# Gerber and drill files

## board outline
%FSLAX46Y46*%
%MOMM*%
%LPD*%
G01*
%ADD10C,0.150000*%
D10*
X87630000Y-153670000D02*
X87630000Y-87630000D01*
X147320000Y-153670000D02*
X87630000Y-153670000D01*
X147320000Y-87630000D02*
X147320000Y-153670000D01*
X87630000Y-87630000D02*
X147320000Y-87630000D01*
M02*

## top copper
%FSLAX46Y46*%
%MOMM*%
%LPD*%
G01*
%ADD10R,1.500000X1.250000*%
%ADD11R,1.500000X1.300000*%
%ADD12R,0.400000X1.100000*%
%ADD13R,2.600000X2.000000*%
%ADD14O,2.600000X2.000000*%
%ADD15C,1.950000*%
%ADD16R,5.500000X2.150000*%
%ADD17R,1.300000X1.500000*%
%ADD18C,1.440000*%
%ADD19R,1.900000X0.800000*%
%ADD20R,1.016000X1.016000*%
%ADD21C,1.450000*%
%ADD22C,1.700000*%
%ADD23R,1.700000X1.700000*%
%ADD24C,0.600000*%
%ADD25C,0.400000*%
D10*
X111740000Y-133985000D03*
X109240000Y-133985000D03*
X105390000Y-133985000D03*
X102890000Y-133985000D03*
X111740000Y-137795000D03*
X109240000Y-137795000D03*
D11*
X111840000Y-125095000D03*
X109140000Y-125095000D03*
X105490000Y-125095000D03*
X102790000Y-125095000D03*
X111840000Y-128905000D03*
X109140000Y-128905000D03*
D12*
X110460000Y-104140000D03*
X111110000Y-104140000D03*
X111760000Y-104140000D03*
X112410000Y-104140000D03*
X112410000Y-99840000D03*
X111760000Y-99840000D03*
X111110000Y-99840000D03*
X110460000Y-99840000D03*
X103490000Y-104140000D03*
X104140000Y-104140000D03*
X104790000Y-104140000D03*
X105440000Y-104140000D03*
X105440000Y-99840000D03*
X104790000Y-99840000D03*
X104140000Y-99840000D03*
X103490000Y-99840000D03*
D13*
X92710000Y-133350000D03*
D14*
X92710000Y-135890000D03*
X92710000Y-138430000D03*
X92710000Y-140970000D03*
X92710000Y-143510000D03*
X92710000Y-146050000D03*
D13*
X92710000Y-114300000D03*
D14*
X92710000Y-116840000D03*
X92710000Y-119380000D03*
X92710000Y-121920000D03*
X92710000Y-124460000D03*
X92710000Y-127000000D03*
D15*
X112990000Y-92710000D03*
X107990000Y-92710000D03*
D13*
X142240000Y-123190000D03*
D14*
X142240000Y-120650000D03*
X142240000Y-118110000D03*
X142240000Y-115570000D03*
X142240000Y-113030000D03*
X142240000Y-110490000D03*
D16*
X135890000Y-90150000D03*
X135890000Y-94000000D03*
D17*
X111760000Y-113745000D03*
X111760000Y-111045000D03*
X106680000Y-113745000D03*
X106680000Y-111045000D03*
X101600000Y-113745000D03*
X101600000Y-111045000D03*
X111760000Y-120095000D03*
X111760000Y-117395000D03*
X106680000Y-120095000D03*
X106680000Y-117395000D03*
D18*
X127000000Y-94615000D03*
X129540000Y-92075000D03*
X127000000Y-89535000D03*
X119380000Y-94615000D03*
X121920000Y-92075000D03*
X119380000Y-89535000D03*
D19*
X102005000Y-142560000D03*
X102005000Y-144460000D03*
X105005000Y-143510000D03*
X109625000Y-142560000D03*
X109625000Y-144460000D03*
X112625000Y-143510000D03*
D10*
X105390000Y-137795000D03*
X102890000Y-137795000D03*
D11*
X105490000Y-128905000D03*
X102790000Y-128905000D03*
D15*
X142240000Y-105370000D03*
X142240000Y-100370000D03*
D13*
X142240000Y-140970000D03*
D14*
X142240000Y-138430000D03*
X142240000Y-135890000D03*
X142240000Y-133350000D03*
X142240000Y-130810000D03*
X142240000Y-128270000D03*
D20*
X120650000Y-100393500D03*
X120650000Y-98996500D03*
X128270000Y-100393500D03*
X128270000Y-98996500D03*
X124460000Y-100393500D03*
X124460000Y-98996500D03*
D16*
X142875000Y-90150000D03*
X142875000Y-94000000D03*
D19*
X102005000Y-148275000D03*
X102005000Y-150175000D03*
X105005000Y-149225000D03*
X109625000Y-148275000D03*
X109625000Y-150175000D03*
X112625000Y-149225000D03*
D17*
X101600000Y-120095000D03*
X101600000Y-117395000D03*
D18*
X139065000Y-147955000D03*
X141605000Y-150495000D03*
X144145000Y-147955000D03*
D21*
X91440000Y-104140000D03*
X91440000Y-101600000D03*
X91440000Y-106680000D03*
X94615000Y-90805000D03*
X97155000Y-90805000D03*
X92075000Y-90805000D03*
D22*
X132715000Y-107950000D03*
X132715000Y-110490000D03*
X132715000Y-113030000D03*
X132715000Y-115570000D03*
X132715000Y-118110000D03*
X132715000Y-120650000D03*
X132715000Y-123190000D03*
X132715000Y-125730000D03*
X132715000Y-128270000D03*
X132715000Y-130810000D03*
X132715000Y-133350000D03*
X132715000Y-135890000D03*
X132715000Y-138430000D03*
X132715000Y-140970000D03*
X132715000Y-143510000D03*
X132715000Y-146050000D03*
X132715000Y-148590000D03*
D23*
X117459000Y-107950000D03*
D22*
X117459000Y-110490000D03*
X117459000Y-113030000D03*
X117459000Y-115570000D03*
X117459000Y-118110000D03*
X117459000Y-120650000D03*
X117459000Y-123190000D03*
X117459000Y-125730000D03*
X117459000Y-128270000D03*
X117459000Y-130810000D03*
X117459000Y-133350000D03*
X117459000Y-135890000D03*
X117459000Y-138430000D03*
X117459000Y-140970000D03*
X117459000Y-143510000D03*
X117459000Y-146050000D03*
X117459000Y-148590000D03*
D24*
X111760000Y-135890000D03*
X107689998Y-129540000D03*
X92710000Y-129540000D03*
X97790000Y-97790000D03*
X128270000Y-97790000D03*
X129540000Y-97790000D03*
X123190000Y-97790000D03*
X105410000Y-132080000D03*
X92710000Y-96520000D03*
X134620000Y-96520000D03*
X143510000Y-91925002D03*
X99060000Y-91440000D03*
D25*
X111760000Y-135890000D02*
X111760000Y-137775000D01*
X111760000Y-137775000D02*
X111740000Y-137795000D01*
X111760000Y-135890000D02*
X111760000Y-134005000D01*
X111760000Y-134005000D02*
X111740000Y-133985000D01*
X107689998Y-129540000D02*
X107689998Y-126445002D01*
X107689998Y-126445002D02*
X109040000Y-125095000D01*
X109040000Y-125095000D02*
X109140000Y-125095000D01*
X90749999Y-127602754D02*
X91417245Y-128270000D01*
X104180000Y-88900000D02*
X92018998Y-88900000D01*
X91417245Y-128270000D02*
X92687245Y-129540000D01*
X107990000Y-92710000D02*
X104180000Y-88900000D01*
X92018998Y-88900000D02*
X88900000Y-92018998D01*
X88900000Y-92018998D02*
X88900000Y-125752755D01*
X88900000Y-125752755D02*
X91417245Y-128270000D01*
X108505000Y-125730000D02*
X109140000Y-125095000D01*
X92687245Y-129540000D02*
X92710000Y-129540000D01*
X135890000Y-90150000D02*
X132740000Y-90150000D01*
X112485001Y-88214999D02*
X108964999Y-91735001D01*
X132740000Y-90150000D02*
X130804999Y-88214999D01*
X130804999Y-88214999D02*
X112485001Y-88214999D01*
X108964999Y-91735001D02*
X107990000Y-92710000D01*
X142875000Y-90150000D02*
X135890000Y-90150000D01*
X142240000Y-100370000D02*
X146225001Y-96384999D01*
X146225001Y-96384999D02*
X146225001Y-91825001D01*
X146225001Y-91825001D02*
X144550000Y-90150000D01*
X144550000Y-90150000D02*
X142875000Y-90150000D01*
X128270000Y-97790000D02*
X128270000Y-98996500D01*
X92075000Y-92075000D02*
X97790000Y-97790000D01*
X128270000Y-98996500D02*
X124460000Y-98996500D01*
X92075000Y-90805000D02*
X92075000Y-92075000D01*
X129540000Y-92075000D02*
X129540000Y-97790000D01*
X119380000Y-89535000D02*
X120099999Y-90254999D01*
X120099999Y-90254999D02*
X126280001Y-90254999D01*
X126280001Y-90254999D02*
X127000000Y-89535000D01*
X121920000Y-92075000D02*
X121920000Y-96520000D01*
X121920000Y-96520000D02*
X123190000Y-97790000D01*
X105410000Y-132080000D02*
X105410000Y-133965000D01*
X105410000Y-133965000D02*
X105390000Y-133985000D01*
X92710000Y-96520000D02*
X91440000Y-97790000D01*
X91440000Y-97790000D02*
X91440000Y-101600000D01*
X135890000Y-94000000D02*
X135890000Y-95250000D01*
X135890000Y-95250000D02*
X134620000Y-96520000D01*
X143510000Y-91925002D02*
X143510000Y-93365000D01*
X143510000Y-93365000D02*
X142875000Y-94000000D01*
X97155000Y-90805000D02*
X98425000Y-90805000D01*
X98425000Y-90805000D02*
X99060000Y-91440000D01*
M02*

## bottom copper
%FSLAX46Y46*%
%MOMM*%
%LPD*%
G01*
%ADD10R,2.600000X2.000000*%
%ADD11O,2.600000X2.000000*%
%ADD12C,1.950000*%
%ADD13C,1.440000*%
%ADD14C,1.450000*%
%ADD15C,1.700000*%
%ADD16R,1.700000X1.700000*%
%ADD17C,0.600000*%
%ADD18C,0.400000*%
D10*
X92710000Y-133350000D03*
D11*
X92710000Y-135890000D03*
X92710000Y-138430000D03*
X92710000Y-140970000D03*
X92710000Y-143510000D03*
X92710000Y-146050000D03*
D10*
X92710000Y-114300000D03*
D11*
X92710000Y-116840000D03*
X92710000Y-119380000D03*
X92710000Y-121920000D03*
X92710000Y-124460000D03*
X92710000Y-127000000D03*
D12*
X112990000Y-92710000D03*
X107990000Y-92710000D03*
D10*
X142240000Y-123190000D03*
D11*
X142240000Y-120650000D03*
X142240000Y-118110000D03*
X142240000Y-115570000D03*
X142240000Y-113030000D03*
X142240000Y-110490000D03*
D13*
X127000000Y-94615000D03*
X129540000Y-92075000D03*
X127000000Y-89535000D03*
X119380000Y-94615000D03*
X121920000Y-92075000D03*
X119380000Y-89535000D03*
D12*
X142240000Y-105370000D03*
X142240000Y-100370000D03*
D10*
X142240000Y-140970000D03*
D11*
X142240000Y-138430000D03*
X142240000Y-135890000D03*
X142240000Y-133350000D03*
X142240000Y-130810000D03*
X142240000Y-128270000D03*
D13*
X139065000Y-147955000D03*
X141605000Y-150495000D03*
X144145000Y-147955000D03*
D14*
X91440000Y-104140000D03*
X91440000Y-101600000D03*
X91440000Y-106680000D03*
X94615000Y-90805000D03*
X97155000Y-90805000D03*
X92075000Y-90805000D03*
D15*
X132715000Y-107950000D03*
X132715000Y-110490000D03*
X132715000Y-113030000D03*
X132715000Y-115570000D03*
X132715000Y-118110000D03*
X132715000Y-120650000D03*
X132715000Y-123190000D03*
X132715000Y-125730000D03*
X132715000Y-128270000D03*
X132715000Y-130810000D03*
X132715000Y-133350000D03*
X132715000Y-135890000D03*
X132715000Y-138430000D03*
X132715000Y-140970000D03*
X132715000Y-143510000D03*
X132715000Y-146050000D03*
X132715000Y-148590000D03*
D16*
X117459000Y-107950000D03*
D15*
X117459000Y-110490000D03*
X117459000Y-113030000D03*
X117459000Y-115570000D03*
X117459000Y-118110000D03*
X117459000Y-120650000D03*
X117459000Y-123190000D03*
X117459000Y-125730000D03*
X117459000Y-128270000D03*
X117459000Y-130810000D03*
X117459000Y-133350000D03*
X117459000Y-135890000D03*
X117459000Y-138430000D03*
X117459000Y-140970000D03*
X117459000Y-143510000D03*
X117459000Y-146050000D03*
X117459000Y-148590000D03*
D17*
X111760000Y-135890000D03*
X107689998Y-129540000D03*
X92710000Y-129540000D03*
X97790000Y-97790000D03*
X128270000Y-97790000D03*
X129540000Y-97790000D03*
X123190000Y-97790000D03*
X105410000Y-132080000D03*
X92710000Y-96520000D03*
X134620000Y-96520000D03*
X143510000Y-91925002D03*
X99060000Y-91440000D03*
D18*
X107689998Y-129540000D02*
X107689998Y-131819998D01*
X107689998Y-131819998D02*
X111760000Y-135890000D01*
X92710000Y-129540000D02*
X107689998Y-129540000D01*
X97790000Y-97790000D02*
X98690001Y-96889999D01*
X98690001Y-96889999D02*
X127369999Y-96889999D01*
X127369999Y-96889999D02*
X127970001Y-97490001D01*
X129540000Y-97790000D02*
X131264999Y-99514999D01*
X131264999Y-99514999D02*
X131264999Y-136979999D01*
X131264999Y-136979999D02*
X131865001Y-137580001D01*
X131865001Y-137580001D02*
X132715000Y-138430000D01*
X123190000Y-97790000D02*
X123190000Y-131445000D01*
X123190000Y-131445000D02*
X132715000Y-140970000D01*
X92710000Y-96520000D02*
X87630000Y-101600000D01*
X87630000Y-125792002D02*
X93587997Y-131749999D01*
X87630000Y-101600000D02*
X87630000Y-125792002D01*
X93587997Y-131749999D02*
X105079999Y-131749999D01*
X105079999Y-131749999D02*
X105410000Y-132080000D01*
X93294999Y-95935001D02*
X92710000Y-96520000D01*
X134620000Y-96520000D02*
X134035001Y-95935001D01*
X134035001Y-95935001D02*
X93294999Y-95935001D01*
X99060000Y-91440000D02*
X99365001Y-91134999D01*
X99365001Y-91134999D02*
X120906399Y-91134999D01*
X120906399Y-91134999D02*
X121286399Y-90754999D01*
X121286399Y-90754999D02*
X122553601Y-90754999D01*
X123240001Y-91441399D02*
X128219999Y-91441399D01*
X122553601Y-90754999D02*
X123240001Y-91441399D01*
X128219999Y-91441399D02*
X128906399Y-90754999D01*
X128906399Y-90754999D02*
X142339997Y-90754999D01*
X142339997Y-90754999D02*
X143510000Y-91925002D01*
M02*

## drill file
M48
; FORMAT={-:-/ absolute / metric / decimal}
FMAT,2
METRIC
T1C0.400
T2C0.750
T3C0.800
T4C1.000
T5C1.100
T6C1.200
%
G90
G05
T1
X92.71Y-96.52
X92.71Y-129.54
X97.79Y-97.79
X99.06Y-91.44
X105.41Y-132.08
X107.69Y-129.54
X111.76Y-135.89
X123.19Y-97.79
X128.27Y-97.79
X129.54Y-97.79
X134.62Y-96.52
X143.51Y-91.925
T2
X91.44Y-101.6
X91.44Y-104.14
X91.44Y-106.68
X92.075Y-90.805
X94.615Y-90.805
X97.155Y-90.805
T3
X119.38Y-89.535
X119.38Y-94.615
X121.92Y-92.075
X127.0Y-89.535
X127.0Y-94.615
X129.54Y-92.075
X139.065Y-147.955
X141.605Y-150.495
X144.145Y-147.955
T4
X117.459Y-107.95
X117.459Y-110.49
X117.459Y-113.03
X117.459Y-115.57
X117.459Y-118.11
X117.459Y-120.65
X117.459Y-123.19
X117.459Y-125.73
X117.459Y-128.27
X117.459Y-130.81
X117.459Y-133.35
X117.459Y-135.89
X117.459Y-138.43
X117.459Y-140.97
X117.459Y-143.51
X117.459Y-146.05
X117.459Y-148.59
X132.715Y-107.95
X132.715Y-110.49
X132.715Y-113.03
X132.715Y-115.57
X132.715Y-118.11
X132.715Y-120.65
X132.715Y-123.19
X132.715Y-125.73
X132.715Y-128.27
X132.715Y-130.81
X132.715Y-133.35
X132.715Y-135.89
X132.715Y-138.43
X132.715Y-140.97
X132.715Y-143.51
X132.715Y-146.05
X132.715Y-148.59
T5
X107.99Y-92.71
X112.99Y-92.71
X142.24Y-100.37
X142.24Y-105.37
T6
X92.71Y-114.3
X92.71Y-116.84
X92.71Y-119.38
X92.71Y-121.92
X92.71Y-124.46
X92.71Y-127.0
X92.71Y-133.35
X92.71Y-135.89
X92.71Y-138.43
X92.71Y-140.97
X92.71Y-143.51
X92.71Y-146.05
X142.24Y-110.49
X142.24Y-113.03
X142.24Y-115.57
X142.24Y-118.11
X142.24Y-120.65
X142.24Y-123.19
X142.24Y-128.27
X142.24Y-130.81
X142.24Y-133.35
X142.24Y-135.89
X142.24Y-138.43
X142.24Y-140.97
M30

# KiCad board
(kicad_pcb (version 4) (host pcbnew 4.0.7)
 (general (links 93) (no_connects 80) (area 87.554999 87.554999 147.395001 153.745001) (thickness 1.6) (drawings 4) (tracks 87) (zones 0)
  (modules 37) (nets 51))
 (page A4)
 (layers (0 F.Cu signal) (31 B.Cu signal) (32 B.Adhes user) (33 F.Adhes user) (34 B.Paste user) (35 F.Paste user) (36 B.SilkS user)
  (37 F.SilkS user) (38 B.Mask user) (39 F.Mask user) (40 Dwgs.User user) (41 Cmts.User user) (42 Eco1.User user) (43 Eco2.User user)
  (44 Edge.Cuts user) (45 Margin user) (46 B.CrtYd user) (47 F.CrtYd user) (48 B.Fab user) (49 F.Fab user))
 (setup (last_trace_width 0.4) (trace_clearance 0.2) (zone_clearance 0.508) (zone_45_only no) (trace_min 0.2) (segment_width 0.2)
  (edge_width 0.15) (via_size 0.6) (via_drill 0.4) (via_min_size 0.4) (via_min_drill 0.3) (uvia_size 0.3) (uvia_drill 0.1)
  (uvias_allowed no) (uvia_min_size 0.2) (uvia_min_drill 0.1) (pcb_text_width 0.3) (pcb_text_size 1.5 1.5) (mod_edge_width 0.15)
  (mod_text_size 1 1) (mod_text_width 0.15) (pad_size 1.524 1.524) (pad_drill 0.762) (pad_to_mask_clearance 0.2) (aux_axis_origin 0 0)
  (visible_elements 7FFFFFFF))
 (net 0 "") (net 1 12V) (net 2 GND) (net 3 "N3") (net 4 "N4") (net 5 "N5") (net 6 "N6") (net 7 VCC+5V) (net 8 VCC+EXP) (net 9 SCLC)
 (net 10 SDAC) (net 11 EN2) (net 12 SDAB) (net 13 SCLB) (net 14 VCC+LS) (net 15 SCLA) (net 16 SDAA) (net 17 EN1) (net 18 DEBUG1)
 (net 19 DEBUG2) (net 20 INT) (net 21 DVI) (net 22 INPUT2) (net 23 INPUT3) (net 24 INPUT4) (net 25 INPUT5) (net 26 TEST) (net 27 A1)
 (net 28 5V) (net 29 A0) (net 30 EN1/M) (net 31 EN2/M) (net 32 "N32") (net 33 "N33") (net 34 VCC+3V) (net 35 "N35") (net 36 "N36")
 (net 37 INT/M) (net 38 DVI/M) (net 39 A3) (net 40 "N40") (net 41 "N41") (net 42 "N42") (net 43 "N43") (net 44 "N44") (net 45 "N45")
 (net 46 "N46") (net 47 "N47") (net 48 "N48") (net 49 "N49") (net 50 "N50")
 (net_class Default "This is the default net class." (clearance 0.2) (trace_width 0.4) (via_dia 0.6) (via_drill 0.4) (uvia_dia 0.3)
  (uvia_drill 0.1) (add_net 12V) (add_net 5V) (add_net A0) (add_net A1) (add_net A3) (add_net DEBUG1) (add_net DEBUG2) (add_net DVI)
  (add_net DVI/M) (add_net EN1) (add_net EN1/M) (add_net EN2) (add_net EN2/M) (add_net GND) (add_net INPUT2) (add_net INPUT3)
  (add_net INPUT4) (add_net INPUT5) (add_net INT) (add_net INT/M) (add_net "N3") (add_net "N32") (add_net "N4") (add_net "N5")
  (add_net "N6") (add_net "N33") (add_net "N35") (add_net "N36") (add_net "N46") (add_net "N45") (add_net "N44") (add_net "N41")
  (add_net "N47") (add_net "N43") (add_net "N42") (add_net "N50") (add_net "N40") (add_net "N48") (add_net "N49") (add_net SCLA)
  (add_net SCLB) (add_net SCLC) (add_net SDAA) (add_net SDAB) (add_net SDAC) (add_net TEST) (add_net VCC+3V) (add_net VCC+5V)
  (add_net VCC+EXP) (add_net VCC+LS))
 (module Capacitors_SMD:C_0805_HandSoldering (layer F.Cu) (at 110.49 133.985 180)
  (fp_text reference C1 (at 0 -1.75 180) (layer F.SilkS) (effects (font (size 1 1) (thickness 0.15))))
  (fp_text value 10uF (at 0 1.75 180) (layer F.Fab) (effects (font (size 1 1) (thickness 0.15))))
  (pad 1 smd rect (at -1.25 0 180) (size 1.5 1.25) (layers F.Cu F.Paste F.Mask) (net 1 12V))
  (pad 2 smd rect (at 1.25 0 180) (size 1.5 1.25) (layers F.Cu F.Paste F.Mask) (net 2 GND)))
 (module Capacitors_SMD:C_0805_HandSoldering (layer F.Cu) (at 104.14 133.985 180)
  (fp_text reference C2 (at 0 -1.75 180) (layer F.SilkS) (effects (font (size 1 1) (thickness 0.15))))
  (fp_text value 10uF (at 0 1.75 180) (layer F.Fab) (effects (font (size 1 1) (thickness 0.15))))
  (pad 1 smd rect (at -1.25 0 180) (size 1.5 1.25) (layers F.Cu F.Paste F.Mask) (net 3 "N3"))
  (pad 2 smd rect (at 1.25 0 180) (size 1.5 1.25) (layers F.Cu F.Paste F.Mask) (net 2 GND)))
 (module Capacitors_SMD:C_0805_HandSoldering (layer F.Cu) (at 110.49 137.795 180)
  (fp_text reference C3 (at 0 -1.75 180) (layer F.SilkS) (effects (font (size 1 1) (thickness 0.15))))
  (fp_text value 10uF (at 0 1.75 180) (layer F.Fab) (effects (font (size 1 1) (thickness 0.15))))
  (pad 1 smd rect (at -1.25 0 180) (size 1.5 1.25) (layers F.Cu F.Paste F.Mask) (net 1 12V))
  (pad 2 smd rect (at 1.25 0 180) (size 1.5 1.25) (layers F.Cu F.Paste F.Mask) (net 2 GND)))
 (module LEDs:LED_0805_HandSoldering (layer F.Cu) (at 110.49 125.095 180)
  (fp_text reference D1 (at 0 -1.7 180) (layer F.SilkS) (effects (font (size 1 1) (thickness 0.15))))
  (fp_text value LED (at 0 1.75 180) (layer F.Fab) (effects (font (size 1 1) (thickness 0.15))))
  (pad 1 smd rect (at -1.35 0 180) (size 1.5 1.3) (layers F.Cu F.Paste F.Mask) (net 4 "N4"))
  (pad 2 smd rect (at 1.35 0 180) (size 1.5 1.3) (layers F.Cu F.Paste F.Mask) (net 1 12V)))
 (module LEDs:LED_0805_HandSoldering (layer F.Cu) (at 104.14 125.095 180)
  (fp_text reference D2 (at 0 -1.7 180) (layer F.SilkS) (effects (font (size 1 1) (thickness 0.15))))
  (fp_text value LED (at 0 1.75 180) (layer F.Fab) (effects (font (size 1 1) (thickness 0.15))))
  (pad 1 smd rect (at -1.35 0 180) (size 1.5 1.3) (layers F.Cu F.Paste F.Mask) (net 2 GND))
  (pad 2 smd rect (at 1.35 0 180) (size 1.5 1.3) (layers F.Cu F.Paste F.Mask) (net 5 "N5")))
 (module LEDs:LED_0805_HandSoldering (layer F.Cu) (at 110.49 128.905 180)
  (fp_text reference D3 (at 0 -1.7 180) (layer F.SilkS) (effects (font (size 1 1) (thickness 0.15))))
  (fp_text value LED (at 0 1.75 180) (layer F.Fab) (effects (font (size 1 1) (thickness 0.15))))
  (pad 1 smd rect (at -1.35 0 180) (size 1.5 1.3) (layers F.Cu F.Paste F.Mask) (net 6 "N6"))
  (pad 2 smd rect (at 1.35 0 180) (size 1.5 1.3) (layers F.Cu F.Paste F.Mask) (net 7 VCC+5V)))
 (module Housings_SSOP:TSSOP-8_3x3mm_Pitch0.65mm (layer F.Cu) (at 111.435 101.99 90)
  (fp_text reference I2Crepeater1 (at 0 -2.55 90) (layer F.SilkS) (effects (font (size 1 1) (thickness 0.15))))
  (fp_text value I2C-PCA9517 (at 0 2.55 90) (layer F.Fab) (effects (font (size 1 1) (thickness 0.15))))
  (pad 1 smd rect (at -2.15 -0.975 90) (size 1.1 0.4) (layers F.Cu F.Paste F.Mask) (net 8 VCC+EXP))
  (pad 2 smd rect (at -2.15 -0.325 90) (size 1.1 0.4) (layers F.Cu F.Paste F.Mask) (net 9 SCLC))
  (pad 3 smd rect (at -2.15 0.325 90) (size 1.1 0.4) (layers F.Cu F.Paste F.Mask) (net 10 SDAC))
  (pad 4 smd rect (at -2.15 0.975 90) (size 1.1 0.4) (layers F.Cu F.Paste F.Mask) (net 2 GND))
  (pad 5 smd rect (at 2.15 0.975 90) (size 1.1 0.4) (layers F.Cu F.Paste F.Mask) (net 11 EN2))
  (pad 6 smd rect (at 2.15 0.325 90) (size 1.1 0.4) (layers F.Cu F.Paste F.Mask) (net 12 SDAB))
  (pad 7 smd rect (at 2.15 -0.325 90) (size 1.1 0.4) (layers F.Cu F.Paste F.Mask) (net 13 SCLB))
  (pad 8 smd rect (at 2.15 -0.975 90) (size 1.1 0.4) (layers F.Cu F.Paste F.Mask) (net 7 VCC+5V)))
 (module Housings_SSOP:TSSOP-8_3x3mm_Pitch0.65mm (layer F.Cu) (at 104.465 101.99 90)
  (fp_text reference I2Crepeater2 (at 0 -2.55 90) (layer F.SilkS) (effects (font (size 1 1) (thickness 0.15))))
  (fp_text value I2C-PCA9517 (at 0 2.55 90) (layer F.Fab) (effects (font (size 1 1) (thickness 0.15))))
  (pad 1 smd rect (at -2.15 -0.975 90) (size 1.1 0.4) (layers F.Cu F.Paste F.Mask) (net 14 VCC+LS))
  (pad 2 smd rect (at -2.15 -0.325 90) (size 1.1 0.4) (layers F.Cu F.Paste F.Mask) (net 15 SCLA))
  (pad 3 smd rect (at -2.15 0.325 90) (size 1.1 0.4) (layers F.Cu F.Paste F.Mask) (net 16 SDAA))
  (pad 4 smd rect (at -2.15 0.975 90) (size 1.1 0.4) (layers F.Cu F.Paste F.Mask) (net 2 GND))
  (pad 5 smd rect (at 2.15 0.975 90) (size 1.1 0.4) (layers F.Cu F.Paste F.Mask) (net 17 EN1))
  (pad 6 smd rect (at 2.15 0.325 90) (size 1.1 0.4) (layers F.Cu F.Paste F.Mask) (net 12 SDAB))
  (pad 7 smd rect (at 2.15 -0.325 90) (size 1.1 0.4) (layers F.Cu F.Paste F.Mask) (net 13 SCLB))
  (pad 8 smd rect (at 2.15 -0.975 90) (size 1.1 0.4) (layers F.Cu F.Paste F.Mask) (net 7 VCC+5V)))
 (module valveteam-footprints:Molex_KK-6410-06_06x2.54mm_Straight (layer F.Cu) (at 92.71 133.35 270)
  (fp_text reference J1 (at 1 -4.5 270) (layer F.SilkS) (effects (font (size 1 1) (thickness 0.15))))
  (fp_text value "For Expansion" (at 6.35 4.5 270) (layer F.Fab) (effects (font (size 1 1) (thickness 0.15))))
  (pad 1 thru_hole rect (at 0 0 270) (size 2 2.6) (drill 1.2) (layers *.Cu *.Mask) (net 8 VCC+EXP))
  (pad 2 thru_hole oval (at 2.54 0 270) (size 2 2.6) (drill 1.2) (layers *.Cu *.Mask) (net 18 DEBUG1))
  (pad 3 thru_hole oval (at 5.08 0 270) (size 2 2.6) (drill 1.2) (layers *.Cu *.Mask) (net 10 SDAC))
  (pad 4 thru_hole oval (at 7.62 0 270) (size 2 2.6) (drill 1.2) (layers *.Cu *.Mask) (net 9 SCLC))
  (pad 5 thru_hole oval (at 10.16 0 270) (size 2 2.6) (drill 1.2) (layers *.Cu *.Mask) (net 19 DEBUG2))
  (pad 6 thru_hole oval (at 12.7 0 270) (size 2 2.6) (drill 1.2) (layers *.Cu *.Mask) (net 2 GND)))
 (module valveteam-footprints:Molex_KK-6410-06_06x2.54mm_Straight (layer F.Cu) (at 92.71 114.3 270)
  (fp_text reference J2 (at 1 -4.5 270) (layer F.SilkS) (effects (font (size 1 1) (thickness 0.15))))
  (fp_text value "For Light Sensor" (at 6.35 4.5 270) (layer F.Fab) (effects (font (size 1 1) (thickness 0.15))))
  (pad 1 thru_hole rect (at 0 0 270) (size 2 2.6) (drill 1.2) (layers *.Cu *.Mask) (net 14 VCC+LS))
  (pad 2 thru_hole oval (at 2.54 0 270) (size 2 2.6) (drill 1.2) (layers *.Cu *.Mask) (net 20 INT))
  (pad 3 thru_hole oval (at 5.08 0 270) (size 2 2.6) (drill 1.2) (layers *.Cu *.Mask) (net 16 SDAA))
  (pad 4 thru_hole oval (at 7.62 0 270) (size 2 2.6) (drill 1.2) (layers *.Cu *.Mask) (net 15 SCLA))
  (pad 5 thru_hole oval (at 10.16 0 270) (size 2 2.6) (drill 1.2) (layers *.Cu *.Mask) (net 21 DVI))
  (pad 6 thru_hole oval (at 12.7 0 270) (size 2 2.6) (drill 1.2) (layers *.Cu *.Mask) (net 2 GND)))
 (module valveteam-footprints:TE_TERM (layer F.Cu) (at 110.49 92.71)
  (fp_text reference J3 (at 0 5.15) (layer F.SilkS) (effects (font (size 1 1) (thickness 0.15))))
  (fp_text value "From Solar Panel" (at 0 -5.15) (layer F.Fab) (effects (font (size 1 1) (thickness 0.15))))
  (pad 2 thru_hole circle (at 2.5 0) (size 1.95 1.95) (drill 1.1) (layers *.Cu *.Mask F.SilkS) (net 2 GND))
  (pad 1 thru_hole circle (at -2.5 0) (size 1.95 1.95) (drill 1.1) (layers *.Cu *.Mask F.SilkS) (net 1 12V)))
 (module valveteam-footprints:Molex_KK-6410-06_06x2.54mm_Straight (layer F.Cu) (at 142.24 123.19 90)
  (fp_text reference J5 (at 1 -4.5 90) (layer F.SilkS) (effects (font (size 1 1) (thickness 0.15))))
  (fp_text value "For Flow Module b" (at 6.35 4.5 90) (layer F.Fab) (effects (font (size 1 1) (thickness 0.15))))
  (pad 1 thru_hole rect (at 0 0 90) (size 2 2.6) (drill 1.2) (layers *.Cu *.Mask) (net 7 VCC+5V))
  (pad 2 thru_hole oval (at 2.54 0 90) (size 2 2.6) (drill 1.2) (layers *.Cu *.Mask) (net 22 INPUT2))
  (pad 3 thru_hole oval (at 5.08 0 90) (size 2 2.6) (drill 1.2) (layers *.Cu *.Mask) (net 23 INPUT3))
  (pad 4 thru_hole oval (at 7.62 0 90) (size 2 2.6) (drill 1.2) (layers *.Cu *.Mask) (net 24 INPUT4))
  (pad 5 thru_hole oval (at 10.16 0 90) (size 2 2.6) (drill 1.2) (layers *.Cu *.Mask) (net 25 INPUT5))
  (pad 6 thru_hole oval (at 12.7 0 90) (size 2 2.6) (drill 1.2) (layers *.Cu *.Mask) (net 2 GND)))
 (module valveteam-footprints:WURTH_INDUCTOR (layer F.Cu) (at 135.89 92.075)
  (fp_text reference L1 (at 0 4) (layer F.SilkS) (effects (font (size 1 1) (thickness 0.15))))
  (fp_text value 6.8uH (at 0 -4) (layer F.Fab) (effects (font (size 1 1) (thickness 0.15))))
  (pad 1 smd rect (at 0 -1.925) (size 5.5 2.15) (layers F.Cu F.Paste F.Mask) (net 1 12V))
  (pad 2 smd rect (at 0 1.925) (size 5.5 2.15) (layers F.Cu F.Paste F.Mask) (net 3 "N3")))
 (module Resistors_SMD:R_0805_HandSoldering (layer F.Cu) (at 111.76 112.395 90)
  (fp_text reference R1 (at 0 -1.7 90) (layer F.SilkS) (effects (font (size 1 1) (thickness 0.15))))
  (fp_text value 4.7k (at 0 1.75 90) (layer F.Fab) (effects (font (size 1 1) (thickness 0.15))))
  (pad 1 smd rect (at -1.35 0 90) (size 1.5 1.3) (layers F.Cu F.Paste F.Mask) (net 7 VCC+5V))
  (pad 2 smd rect (at 1.35 0 90) (size 1.5 1.3) (layers F.Cu F.Paste F.Mask) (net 13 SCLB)))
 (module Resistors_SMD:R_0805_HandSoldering (layer F.Cu) (at 106.68 112.395 90)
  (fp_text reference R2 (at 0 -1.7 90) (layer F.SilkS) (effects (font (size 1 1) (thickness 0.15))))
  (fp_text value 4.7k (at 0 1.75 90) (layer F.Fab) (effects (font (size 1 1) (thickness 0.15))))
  (pad 1 smd rect (at -1.35 0 90) (size 1.5 1.3) (layers F.Cu F.Paste F.Mask) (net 7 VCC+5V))
  (pad 2 smd rect (at 1.35 0 90) (size 1.5 1.3) (layers F.Cu F.Paste F.Mask) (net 12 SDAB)))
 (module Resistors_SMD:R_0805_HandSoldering (layer F.Cu) (at 101.6 112.395 90)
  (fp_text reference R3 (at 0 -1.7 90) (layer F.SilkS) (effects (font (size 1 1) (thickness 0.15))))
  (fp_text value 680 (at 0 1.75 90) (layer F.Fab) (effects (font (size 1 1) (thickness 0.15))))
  (pad 1 smd rect (at -1.35 0 90) (size 1.5 1.3) (layers F.Cu F.Paste F.Mask) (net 4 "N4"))
  (pad 2 smd rect (at 1.35 0 90) (size 1.5 1.3) (layers F.Cu F.Paste F.Mask) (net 2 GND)))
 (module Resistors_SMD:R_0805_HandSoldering (layer F.Cu) (at 111.76 118.745 90)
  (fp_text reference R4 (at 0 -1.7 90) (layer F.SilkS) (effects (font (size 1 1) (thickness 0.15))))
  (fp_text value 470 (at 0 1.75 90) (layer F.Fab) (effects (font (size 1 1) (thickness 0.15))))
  (pad 1 smd rect (at -1.35 0 90) (size 1.5 1.3) (layers F.Cu F.Paste F.Mask) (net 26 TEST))
  (pad 2 smd rect (at 1.35 0 90) (size 1.5 1.3) (layers F.Cu F.Paste F.Mask) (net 5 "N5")))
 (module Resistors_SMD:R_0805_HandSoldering (layer F.Cu) (at 106.68 118.745 90)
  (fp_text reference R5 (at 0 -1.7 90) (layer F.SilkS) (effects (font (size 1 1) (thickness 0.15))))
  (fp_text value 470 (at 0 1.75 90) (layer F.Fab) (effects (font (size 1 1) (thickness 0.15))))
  (pad 1 smd rect (at -1.35 0 90) (size 1.5 1.3) (layers F.Cu F.Paste F.Mask) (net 6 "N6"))
  (pad 2 smd rect (at 1.35 0 90) (size 1.5 1.3) (layers F.Cu F.Paste F.Mask) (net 2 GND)))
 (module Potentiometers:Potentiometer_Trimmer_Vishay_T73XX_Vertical (layer F.Cu) (at 127 89.535)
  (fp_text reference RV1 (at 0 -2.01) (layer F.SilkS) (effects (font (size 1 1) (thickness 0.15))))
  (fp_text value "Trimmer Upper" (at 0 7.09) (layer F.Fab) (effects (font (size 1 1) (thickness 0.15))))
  (pad 3 thru_hole circle (at 0 5.08) (size 1.44 1.44) (drill 0.8) (layers *.Cu *.Mask) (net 2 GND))
  (pad 2 thru_hole circle (at 2.54 2.54) (size 1.44 1.44) (drill 0.8) (layers *.Cu *.Mask) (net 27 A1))
  (pad 1 thru_hole circle (at 0 0) (size 1.44 1.44) (drill 0.8) (layers *.Cu *.Mask) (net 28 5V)))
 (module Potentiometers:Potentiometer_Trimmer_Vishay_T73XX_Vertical (layer F.Cu) (at 119.38 89.535)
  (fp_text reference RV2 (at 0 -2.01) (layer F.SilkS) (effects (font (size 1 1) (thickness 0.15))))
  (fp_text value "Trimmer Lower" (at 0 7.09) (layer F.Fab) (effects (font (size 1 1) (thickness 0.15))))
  (pad 3 thru_hole circle (at 0 5.08) (size 1.44 1.44) (drill 0.8) (layers *.Cu *.Mask) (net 2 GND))
  (pad 2 thru_hole circle (at 2.54 2.54) (size 1.44 1.44) (drill 0.8) (layers *.Cu *.Mask) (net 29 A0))
  (pad 1 thru_hole circle (at 0 0) (size 1.44 1.44) (drill 0.8) (layers *.Cu *.Mask) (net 28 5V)))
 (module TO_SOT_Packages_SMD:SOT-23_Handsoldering (layer F.Cu) (at 103.505 143.51)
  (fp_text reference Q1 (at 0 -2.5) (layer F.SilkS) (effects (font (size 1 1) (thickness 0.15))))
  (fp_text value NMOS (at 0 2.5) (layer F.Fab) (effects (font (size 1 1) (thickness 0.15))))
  (pad 1 smd rect (at -1.5 -0.95) (size 1.9 0.8) (layers F.Cu F.Paste F.Mask) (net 17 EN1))
  (pad 2 smd rect (at -1.5 0.95) (size 1.9 0.8) (layers F.Cu F.Paste F.Mask) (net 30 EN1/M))
  (pad 3 smd rect (at 1.5 0) (size 1.9 0.8) (layers F.Cu F.Paste F.Mask) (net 2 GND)))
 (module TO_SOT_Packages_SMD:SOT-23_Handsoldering (layer F.Cu) (at 111.125 143.51)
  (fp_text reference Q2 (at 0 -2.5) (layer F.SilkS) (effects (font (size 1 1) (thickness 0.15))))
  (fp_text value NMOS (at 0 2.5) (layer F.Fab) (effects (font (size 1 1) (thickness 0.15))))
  (pad 1 smd rect (at -1.5 -0.95) (size 1.9 0.8) (layers F.Cu F.Paste F.Mask) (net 11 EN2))
  (pad 2 smd rect (at -1.5 0.95) (size 1.9 0.8) (layers F.Cu F.Paste F.Mask) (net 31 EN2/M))
  (pad 3 smd rect (at 1.5 0) (size 1.9 0.8) (layers F.Cu F.Paste F.Mask) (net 2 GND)))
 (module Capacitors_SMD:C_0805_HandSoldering (layer F.Cu) (at 104.14 137.795 180)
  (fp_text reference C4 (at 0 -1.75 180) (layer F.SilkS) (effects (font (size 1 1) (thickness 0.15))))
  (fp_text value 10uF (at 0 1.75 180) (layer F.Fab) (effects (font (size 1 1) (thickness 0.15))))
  (pad 1 smd rect (at -1.25 0 180) (size 1.5 1.25) (layers F.Cu F.Paste F.Mask) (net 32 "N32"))
  (pad 2 smd rect (at 1.25 0 180) (size 1.5 1.25) (layers F.Cu F.Paste F.Mask) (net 2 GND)))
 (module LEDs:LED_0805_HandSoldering (layer F.Cu) (at 104.14 128.905 180)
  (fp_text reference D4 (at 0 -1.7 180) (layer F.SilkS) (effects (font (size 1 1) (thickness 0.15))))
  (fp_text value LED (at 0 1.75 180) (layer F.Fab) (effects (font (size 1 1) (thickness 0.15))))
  (pad 1 smd rect (at -1.35 0 180) (size 1.5 1.3) (layers F.Cu F.Paste F.Mask) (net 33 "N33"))
  (pad 2 smd rect (at 1.35 0 180) (size 1.5 1.3) (layers F.Cu F.Paste F.Mask) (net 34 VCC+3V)))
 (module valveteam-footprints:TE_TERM (layer F.Cu) (at 142.24 102.87 270)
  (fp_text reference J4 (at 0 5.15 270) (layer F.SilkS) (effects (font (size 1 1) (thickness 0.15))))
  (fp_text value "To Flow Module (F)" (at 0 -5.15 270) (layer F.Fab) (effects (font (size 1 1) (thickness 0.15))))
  (pad 2 thru_hole circle (at 2.5 0 270) (size 1.95 1.95) (drill 1.1) (layers *.Cu *.Mask F.SilkS) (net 2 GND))
  (pad 1 thru_hole circle (at -2.5 0 270) (size 1.95 1.95) (drill 1.1) (layers *.Cu *.Mask F.SilkS) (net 1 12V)))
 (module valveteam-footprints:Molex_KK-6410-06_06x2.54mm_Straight (layer F.Cu) (at 142.24 140.97 90)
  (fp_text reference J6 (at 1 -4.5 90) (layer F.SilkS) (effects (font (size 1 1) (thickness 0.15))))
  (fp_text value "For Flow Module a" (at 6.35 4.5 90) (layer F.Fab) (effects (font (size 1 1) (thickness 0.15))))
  (pad 1 thru_hole rect (at 0 0 90) (size 2 2.6) (drill 1.2) (layers *.Cu *.Mask) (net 7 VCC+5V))
  (pad 2 thru_hole oval (at 2.54 0 90) (size 2 2.6) (drill 1.2) (layers *.Cu *.Mask) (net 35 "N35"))
  (pad 3 thru_hole oval (at 5.08 0 90) (size 2 2.6) (drill 1.2) (layers *.Cu *.Mask) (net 23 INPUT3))
  (pad 4 thru_hole oval (at 7.62 0 90) (size 2 2.6) (drill 1.2) (layers *.Cu *.Mask) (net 24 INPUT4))
  (pad 5 thru_hole oval (at 10.16 0 90) (size 2 2.6) (drill 1.2) (layers *.Cu *.Mask) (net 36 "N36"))
  (pad 6 thru_hole oval (at 12.7 0 90) (size 2 2.6) (drill 1.2) (layers *.Cu *.Mask) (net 2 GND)))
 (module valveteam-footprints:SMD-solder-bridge (layer F.Cu) (at 120.65 99.695 90)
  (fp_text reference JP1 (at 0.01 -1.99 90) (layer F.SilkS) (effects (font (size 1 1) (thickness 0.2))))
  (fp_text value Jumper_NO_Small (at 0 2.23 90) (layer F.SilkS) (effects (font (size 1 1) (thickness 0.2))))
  (pad 1 smd rect (at -0.6985 0 90) (size 1.016 1.016) (layers F.Cu F.Paste F.Mask) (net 8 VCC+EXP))
  (pad 2 smd rect (at 0.6985 0 90) (size 1.016 1.016) (layers F.Cu F.Paste F.Mask) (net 7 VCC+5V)))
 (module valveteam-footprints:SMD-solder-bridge (layer F.Cu) (at 128.27 99.695 90)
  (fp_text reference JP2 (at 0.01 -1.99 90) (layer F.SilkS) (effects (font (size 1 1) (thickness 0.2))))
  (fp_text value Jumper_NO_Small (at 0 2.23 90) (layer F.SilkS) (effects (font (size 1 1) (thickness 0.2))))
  (pad 1 smd rect (at -0.6985 0 90) (size 1.016 1.016) (layers F.Cu F.Paste F.Mask) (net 8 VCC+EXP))
  (pad 2 smd rect (at 0.6985 0 90) (size 1.016 1.016) (layers F.Cu F.Paste F.Mask) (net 34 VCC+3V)))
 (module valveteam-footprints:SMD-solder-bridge (layer F.Cu) (at 124.46 99.695 90)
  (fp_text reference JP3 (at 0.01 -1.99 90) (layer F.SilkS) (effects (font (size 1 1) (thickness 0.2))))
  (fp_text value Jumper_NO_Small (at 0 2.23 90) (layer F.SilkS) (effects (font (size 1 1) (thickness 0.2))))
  (pad 1 smd rect (at -0.6985 0 90) (size 1.016 1.016) (layers F.Cu F.Paste F.Mask) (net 14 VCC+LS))
  (pad 2 smd rect (at 0.6985 0 90) (size 1.016 1.016) (layers F.Cu F.Paste F.Mask) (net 34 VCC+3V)))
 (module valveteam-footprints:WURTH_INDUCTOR (layer F.Cu) (at 142.875 92.075)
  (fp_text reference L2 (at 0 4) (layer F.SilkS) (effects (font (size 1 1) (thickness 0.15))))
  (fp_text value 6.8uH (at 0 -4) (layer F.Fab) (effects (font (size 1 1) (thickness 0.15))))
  (pad 1 smd rect (at 0 -1.925) (size 5.5 2.15) (layers F.Cu F.Paste F.Mask) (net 1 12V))
  (pad 2 smd rect (at 0 1.925) (size 5.5 2.15) (layers F.Cu F.Paste F.Mask) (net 32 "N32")))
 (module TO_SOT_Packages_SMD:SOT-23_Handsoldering (layer F.Cu) (at 103.505 149.225)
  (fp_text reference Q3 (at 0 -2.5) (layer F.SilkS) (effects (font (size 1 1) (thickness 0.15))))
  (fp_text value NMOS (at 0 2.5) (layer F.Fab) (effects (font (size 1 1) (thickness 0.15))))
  (pad 1 smd rect (at -1.5 -0.95) (size 1.9 0.8) (layers F.Cu F.Paste F.Mask) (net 20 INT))
  (pad 2 smd rect (at -1.5 0.95) (size 1.9 0.8) (layers F.Cu F.Paste F.Mask) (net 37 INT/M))
  (pad 3 smd rect (at 1.5 0) (size 1.9 0.8) (layers F.Cu F.Paste F.Mask) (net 2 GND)))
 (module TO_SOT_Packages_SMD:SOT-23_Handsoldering (layer F.Cu) (at 111.125 149.225)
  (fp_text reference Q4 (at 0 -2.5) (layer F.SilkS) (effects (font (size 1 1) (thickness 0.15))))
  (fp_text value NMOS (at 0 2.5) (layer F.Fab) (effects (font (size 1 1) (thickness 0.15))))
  (pad 1 smd rect (at -1.5 -0.95) (size 1.9 0.8) (layers F.Cu F.Paste F.Mask) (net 21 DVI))
  (pad 2 smd rect (at -1.5 0.95) (size 1.9 0.8) (layers F.Cu F.Paste F.Mask) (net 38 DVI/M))
  (pad 3 smd rect (at 1.5 0) (size 1.9 0.8) (layers F.Cu F.Paste F.Mask) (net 2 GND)))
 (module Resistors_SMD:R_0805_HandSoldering (layer F.Cu) (at 101.6 118.745 90)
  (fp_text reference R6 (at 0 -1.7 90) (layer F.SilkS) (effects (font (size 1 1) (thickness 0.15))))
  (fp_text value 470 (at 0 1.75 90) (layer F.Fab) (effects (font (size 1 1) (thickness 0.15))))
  (pad 1 smd rect (at -1.35 0 90) (size 1.5 1.3) (layers F.Cu F.Paste F.Mask) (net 33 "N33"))
  (pad 2 smd rect (at 1.35 0 90) (size 1.5 1.3) (layers F.Cu F.Paste F.Mask) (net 2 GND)))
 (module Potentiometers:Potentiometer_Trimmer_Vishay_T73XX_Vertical (layer F.Cu) (at 144.145 147.955 270)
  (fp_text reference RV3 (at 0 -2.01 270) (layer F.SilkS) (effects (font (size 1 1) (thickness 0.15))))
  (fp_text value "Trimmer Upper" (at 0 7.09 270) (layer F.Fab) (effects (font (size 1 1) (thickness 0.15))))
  (pad 3 thru_hole circle (at 0 5.08 270) (size 1.44 1.44) (drill 0.8) (layers *.Cu *.Mask) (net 2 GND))
  (pad 2 thru_hole circle (at 2.54 2.54 270) (size 1.44 1.44) (drill 0.8) (layers *.Cu *.Mask) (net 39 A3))
  (pad 1 thru_hole circle (at 0 0 270) (size 1.44 1.44) (drill 0.8) (layers *.Cu *.Mask) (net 28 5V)))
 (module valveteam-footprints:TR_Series (layer F.Cu) (at 91.44 104.14 90)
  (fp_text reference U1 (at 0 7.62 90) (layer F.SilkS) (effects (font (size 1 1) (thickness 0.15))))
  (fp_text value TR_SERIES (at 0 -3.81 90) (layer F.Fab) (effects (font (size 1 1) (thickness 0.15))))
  (pad GND thru_hole circle (at 0 0 90) (size 1.45 1.45) (drill 0.75) (layers *.Cu *.Mask F.SilkS) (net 2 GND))
  (pad VI thru_hole circle (at 2.54 0 90) (size 1.45 1.45) (drill 0.75) (layers *.Cu *.Mask F.SilkS) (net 3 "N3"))
  (pad VO thru_hole circle (at -2.54 0 90) (size 1.45 1.45) (drill 0.75) (layers *.Cu *.Mask F.SilkS) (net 7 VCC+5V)))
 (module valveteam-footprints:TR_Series (layer F.Cu) (at 94.615 90.805)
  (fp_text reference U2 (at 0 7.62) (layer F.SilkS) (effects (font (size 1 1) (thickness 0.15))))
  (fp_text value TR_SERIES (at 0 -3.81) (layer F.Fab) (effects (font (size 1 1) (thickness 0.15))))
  (pad GND thru_hole circle (at 0 0) (size 1.45 1.45) (drill 0.75) (layers *.Cu *.Mask F.SilkS) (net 2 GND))
  (pad VI thru_hole circle (at 2.54 0) (size 1.45 1.45) (drill 0.75) (layers *.Cu *.Mask F.SilkS) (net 32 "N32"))
  (pad VO thru_hole circle (at -2.54 0) (size 1.45 1.45) (drill 0.75) (layers *.Cu *.Mask F.SilkS) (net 34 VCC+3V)))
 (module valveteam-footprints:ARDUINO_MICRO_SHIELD (layer F.Cu) (at 116.205 104.45 270)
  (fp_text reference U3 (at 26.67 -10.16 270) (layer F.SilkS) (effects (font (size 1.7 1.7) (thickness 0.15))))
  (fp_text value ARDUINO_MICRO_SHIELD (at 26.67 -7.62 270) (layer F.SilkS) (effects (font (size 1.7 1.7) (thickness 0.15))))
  (pad SCK thru_hole circle (at 3.5 -16.51 270) (size 1.7 1.7) (drill 1) (layers *.Cu *.Mask) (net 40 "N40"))
  (pad MI thru_hole circle (at 6.04 -16.51 270) (size 1.7 1.7) (drill 1) (layers *.Cu *.Mask) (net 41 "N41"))
  (pad VI thru_hole circle (at 8.58 -16.51 270) (size 1.7 1.7) (drill 1) (layers *.Cu *.Mask) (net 7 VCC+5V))
  (pad GND thru_hole circle (at 11.12 -16.51 270) (size 1.7 1.7) (drill 1) (layers *.Cu *.Mask) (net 2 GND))
  (pad RST thru_hole circle (at 13.66 -16.51 270) (size 1.7 1.7) (drill 1) (layers *.Cu *.Mask) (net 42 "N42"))
  (pad 5V thru_hole circle (at 16.2 -16.51 270) (size 1.7 1.7) (drill 1) (layers *.Cu *.Mask) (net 28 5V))
  (pad NC thru_hole circle (at 18.74 -16.51 270) (size 1.7 1.7) (drill 1) (layers *.Cu *.Mask) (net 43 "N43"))
  (pad NC thru_hole circle (at 21.28 -16.51 270) (size 1.7 1.7) (drill 1) (layers *.Cu *.Mask) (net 43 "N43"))
  (pad A5 thru_hole circle (at 23.82 -16.51 270) (size 1.7 1.7) (drill 1) (layers *.Cu *.Mask) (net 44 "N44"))
  (pad A4 thru_hole circle (at 26.36 -16.51 270) (size 1.7 1.7) (drill 1) (layers *.Cu *.Mask) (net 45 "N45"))
  (pad A3 thru_hole circle (at 28.9 -16.51 270) (size 1.7 1.7) (drill 1) (layers *.Cu *.Mask) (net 39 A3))
  (pad A2 thru_hole circle (at 31.44 -16.51 270) (size 1.7 1.7) (drill 1) (layers *.Cu *.Mask) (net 31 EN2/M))
  (pad A1 thru_hole circle (at 33.98 -16.51 270) (size 1.7 1.7) (drill 1) (layers *.Cu *.Mask) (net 27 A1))
  (pad A0 thru_hole circle (at 36.52 -16.51 270) (size 1.7 1.7) (drill 1) (layers *.Cu *.Mask) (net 29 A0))
  (pad AREF thru_hole circle (at 39.06 -16.51 270) (size 1.7 1.7) (drill 1) (layers *.Cu *.Mask) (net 2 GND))
  (pad 3.3V thru_hole circle (at 41.6 -16.51 270) (size 1.7 1.7) (drill 1) (layers *.Cu *.Mask) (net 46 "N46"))
  (pad 13 thru_hole circle (at 44.14 -16.51 270) (size 1.7 1.7) (drill 1) (layers *.Cu *.Mask) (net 19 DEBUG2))
  (pad MO thru_hole rect (at 3.5 -1.254 270) (size 1.7 1.7) (drill 1) (layers *.Cu *.Mask) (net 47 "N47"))
  (pad SS thru_hole circle (at 6.04 -1.254 270) (size 1.7 1.7) (drill 1) (layers *.Cu *.Mask) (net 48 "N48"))
  (pad TX thru_hole circle (at 8.58 -1.254 270) (size 1.7 1.7) (drill 1) (layers *.Cu *.Mask) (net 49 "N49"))
  (pad RX thru_hole circle (at 11.12 -1.254 270) (size 1.7 1.7) (drill 1) (layers *.Cu *.Mask) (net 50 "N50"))
  (pad RST thru_hole circle (at 13.66 -1.254 270) (size 1.7 1.7) (drill 1) (layers *.Cu *.Mask) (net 42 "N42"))
  (pad GND thru_hole circle (at 16.2 -1.254 270) (size 1.7 1.7) (drill 1) (layers *.Cu *.Mask) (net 2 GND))
  (pad 2 thru_hole circle (at 18.74 -1.254 270) (size 1.7 1.7) (drill 1) (layers *.Cu *.Mask) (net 12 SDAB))
  (pad 3 thru_hole circle (at 21.28 -1.254 270) (size 1.7 1.7) (drill 1) (layers *.Cu *.Mask) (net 13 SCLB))
  (pad 4 thru_hole circle (at 23.82 -1.254 270) (size 1.7 1.7) (drill 1) (layers *.Cu *.Mask) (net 30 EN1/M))
  (pad 5 thru_hole circle (at 26.36 -1.254 270) (size 1.7 1.7) (drill 1) (layers *.Cu *.Mask) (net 26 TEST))
  (pad 6 thru_hole circle (at 28.9 -1.254 270) (size 1.7 1.7) (drill 1) (layers *.Cu *.Mask) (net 37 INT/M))
  (pad 7 thru_hole circle (at 31.44 -1.254 270) (size 1.7 1.7) (drill 1) (layers *.Cu *.Mask) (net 38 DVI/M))
  (pad 8 thru_hole circle (at 33.98 -1.254 270) (size 1.7 1.7) (drill 1) (layers *.Cu *.Mask) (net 22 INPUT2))
  (pad 9 thru_hole circle (at 36.52 -1.254 270) (size 1.7 1.7) (drill 1) (layers *.Cu *.Mask) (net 23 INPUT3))
  (pad 10 thru_hole circle (at 39.06 -1.254 270) (size 1.7 1.7) (drill 1) (layers *.Cu *.Mask) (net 24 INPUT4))
  (pad 11 thru_hole circle (at 41.6 -1.254 270) (size 1.7 1.7) (drill 1) (layers *.Cu *.Mask) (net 25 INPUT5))
  (pad 12 thru_hole circle (at 44.14 -1.254 270) (size 1.7 1.7) (drill 1) (layers *.Cu *.Mask) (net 18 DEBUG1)))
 (gr_line (start 87.63 153.67) (end 87.63 87.63) (layer Edge.Cuts) (width 0.15))
 (gr_line (start 147.32 153.67) (end 87.63 153.67) (layer Edge.Cuts) (width 0.15))
 (gr_line (start 147.32 87.63) (end 147.32 153.67) (layer Edge.Cuts) (width 0.15))
 (gr_line (start 87.63 87.63) (end 147.32 87.63) (layer Edge.Cuts) (width 0.15))
 (segment (start 111.76 135.89) (end 111.76 137.775) (width 0.4) (layer F.Cu) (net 1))
 (segment (start 111.76 137.775) (end 111.74 137.795) (width 0.4) (layer F.Cu) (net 1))
 (segment (start 111.76 135.89) (end 111.76 134.005) (width 0.4) (layer F.Cu) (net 1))
 (segment (start 111.76 134.005) (end 111.74 133.985) (width 0.4) (layer F.Cu) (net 1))
 (segment (start 107.689998 129.54) (end 107.689998 131.819998) (width 0.4) (layer B.Cu) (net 1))
 (segment (start 107.689998 131.819998) (end 111.76 135.89) (width 0.4) (layer B.Cu) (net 1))
 (via (at 111.76 135.89) (size 0.6) (drill 0.4) (layers F.Cu B.Cu) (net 1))
 (segment (start 107.689998 129.54) (end 107.689998 126.445002) (width 0.4) (layer F.Cu) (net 1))
 (segment (start 107.689998 126.445002) (end 109.04 125.095) (width 0.4) (layer F.Cu) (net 1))
 (segment (start 109.04 125.095) (end 109.14 125.095) (width 0.4) (layer F.Cu) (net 1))
 (segment (start 92.71 129.54) (end 107.689998 129.54) (width 0.4) (layer B.Cu) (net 1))
 (via (at 107.689998 129.54) (size 0.6) (drill 0.4) (layers F.Cu B.Cu) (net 1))
 (segment (start 90.749999 127.602754) (end 91.417245 128.27) (width 0.4) (layer F.Cu) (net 1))
 (segment (start 104.18 88.9) (end 92.018998 88.9) (width 0.4) (layer F.Cu) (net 1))
 (segment (start 91.417245 128.27) (end 92.687245 129.54) (width 0.4) (layer F.Cu) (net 1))
 (segment (start 107.99 92.71) (end 104.18 88.9) (width 0.4) (layer F.Cu) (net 1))
 (segment (start 92.018998 88.9) (end 88.9 92.018998) (width 0.4) (layer F.Cu) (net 1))
 (segment (start 88.9 92.018998) (end 88.9 125.752755) (width 0.4) (layer F.Cu) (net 1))
 (segment (start 88.9 125.752755) (end 91.417245 128.27) (width 0.4) (layer F.Cu) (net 1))
 (segment (start 108.505 125.73) (end 109.14 125.095) (width 0.4) (layer F.Cu) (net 1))
 (segment (start 92.687245 129.54) (end 92.71 129.54) (width 0.4) (layer F.Cu) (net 1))
 (via (at 92.71 129.54) (size 0.6) (drill 0.4) (layers F.Cu B.Cu) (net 1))
 (segment (start 135.89 90.15) (end 132.74 90.15) (width 0.4) (layer F.Cu) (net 1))
 (segment (start 112.485001 88.214999) (end 108.964999 91.735001) (width 0.4) (layer F.Cu) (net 1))
 (segment (start 132.74 90.15) (end 130.804999 88.214999) (width 0.4) (layer F.Cu) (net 1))
 (segment (start 130.804999 88.214999) (end 112.485001 88.214999) (width 0.4) (layer F.Cu) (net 1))
 (segment (start 108.964999 91.735001) (end 107.99 92.71) (width 0.4) (layer F.Cu) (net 1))
 (segment (start 142.875 90.15) (end 135.89 90.15) (width 0.4) (layer F.Cu) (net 1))
 (segment (start 142.24 100.37) (end 146.225001 96.384999) (width 0.4) (layer F.Cu) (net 1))
 (segment (start 146.225001 96.384999) (end 146.225001 91.825001) (width 0.4) (layer F.Cu) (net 1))
 (segment (start 146.225001 91.825001) (end 144.55 90.15) (width 0.4) (layer F.Cu) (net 1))
 (segment (start 144.55 90.15) (end 142.875 90.15) (width 0.4) (layer F.Cu) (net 1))
 (segment (start 128.27 97.79) (end 128.27 98.9965) (width 0.4) (layer F.Cu) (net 34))
 (segment (start 97.79 97.79) (end 98.690001 96.889999) (width 0.4) (layer B.Cu) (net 34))
 (segment (start 98.690001 96.889999) (end 127.369999 96.889999) (width 0.4) (layer B.Cu) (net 34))
 (segment (start 127.369999 96.889999) (end 127.970001 97.490001) (width 0.4) (layer B.Cu) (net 34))
 (segment (start 92.075 92.075) (end 97.79 97.79) (width 0.4) (layer F.Cu) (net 34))
 (via (at 97.79 97.79) (size 0.6) (drill 0.4) (layers F.Cu B.Cu) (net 34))
 (segment (start 128.27 98.9965) (end 124.46 98.9965) (width 0.4) (layer F.Cu) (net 34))
 (via (at 128.27 97.79) (size 0.6) (drill 0.4) (layers F.Cu B.Cu) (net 34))
 (segment (start 92.075 90.805) (end 92.075 92.075) (width 0.4) (layer F.Cu) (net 34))
 (segment (start 129.54 97.79) (end 131.264999 99.514999) (width 0.4) (layer B.Cu) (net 27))
 (segment (start 131.264999 99.514999) (end 131.264999 136.979999) (width 0.4) (layer B.Cu) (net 27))
 (segment (start 131.264999 136.979999) (end 131.865001 137.580001) (width 0.4) (layer B.Cu) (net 27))
 (segment (start 131.865001 137.580001) (end 132.715 138.43) (width 0.4) (layer B.Cu) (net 27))
 (via (at 129.54 97.79) (size 0.6) (drill 0.4) (layers F.Cu B.Cu) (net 27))
 (segment (start 129.54 92.075) (end 129.54 97.79) (width 0.4) (layer F.Cu) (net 27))
 (segment (start 119.38 89.535) (end 120.099999 90.254999) (width 0.4) (layer F.Cu) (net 28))
 (segment (start 120.099999 90.254999) (end 126.280001 90.254999) (width 0.4) (layer F.Cu) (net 28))
 (segment (start 126.280001 90.254999) (end 127 89.535) (width 0.4) (layer F.Cu) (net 28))
 (segment (start 123.19 97.79) (end 123.19 131.445) (width 0.4) (layer B.Cu) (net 29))
 (segment (start 123.19 131.445) (end 132.715 140.97) (width 0.4) (layer B.Cu) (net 29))
 (segment (start 121.92 92.075) (end 121.92 96.52) (width 0.4) (layer F.Cu) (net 29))
 (segment (start 121.92 96.52) (end 123.19 97.79) (width 0.4) (layer F.Cu) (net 29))
 (via (at 123.19 97.79) (size 0.6) (drill 0.4) (layers F.Cu B.Cu) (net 29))
 (segment (start 105.41 132.08) (end 105.41 133.965) (width 0.4) (layer F.Cu) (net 3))
 (segment (start 105.41 133.965) (end 105.39 133.985) (width 0.4) (layer F.Cu) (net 3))
 (segment (start 92.71 96.52) (end 87.63 101.6) (width 0.4) (layer B.Cu) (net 3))
 (segment (start 87.63 125.792002) (end 93.587997 131.749999) (width 0.4) (layer B.Cu) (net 3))
 (segment (start 87.63 101.6) (end 87.63 125.792002) (width 0.4) (layer B.Cu) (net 3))
 (segment (start 93.587997 131.749999) (end 105.079999 131.749999) (width 0.4) (layer B.Cu) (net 3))
 (segment (start 105.079999 131.749999) (end 105.41 132.08) (width 0.4) (layer B.Cu) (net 3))
 (via (at 105.41 132.08) (size 0.6) (drill 0.4) (layers F.Cu B.Cu) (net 3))
 (segment (start 92.71 96.52) (end 91.44 97.79) (width 0.4) (layer F.Cu) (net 3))
 (segment (start 91.44 97.79) (end 91.44 101.6) (width 0.4) (layer F.Cu) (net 3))
 (segment (start 93.294999 95.935001) (end 92.71 96.52) (width 0.4) (layer B.Cu) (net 3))
 (via (at 92.71 96.52) (size 0.6) (drill 0.4) (layers F.Cu B.Cu) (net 3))
 (segment (start 134.62 96.52) (end 134.035001 95.935001) (width 0.4) (layer B.Cu) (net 3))
 (segment (start 134.035001 95.935001) (end 93.294999 95.935001) (width 0.4) (layer B.Cu) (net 3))
 (segment (start 135.89 94) (end 135.89 95.25) (width 0.4) (layer F.Cu) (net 3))
 (segment (start 135.89 95.25) (end 134.62 96.52) (width 0.4) (layer F.Cu) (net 3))
 (via (at 134.62 96.52) (size 0.6) (drill 0.4) (layers F.Cu B.Cu) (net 3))
 (segment (start 143.51 91.925002) (end 143.51 93.365) (width 0.4) (layer F.Cu) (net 32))
 (segment (start 143.51 93.365) (end 142.875 94) (width 0.4) (layer F.Cu) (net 32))
 (segment (start 99.06 91.44) (end 99.365001 91.134999) (width 0.4) (layer B.Cu) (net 32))
 (segment (start 99.365001 91.134999) (end 120.906399 91.134999) (width 0.4) (layer B.Cu) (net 32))
 (segment (start 120.906399 91.134999) (end 121.286399 90.754999) (width 0.4) (layer B.Cu) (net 32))
 (segment (start 121.286399 90.754999) (end 122.553601 90.754999) (width 0.4) (layer B.Cu) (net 32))
 (segment (start 123.240001 91.441399) (end 128.219999 91.441399) (width 0.4) (layer B.Cu) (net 32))
 (segment (start 122.553601 90.754999) (end 123.240001 91.441399) (width 0.4) (layer B.Cu) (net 32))
 (segment (start 128.219999 91.441399) (end 128.906399 90.754999) (width 0.4) (layer B.Cu) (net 32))
 (segment (start 128.906399 90.754999) (end 142.339997 90.754999) (width 0.4) (layer B.Cu) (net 32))
 (segment (start 142.339997 90.754999) (end 143.51 91.925002) (width 0.4) (layer B.Cu) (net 32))
 (via (at 143.51 91.925002) (size 0.6) (drill 0.4) (layers F.Cu B.Cu) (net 32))
 (segment (start 97.155 90.805) (end 98.425 90.805) (width 0.4) (layer F.Cu) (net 32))
 (segment (start 98.425 90.805) (end 99.06 91.44) (width 0.4) (layer F.Cu) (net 32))
 (via (at 99.06 91.44) (size 0.6) (drill 0.4) (layers F.Cu B.Cu) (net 32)))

